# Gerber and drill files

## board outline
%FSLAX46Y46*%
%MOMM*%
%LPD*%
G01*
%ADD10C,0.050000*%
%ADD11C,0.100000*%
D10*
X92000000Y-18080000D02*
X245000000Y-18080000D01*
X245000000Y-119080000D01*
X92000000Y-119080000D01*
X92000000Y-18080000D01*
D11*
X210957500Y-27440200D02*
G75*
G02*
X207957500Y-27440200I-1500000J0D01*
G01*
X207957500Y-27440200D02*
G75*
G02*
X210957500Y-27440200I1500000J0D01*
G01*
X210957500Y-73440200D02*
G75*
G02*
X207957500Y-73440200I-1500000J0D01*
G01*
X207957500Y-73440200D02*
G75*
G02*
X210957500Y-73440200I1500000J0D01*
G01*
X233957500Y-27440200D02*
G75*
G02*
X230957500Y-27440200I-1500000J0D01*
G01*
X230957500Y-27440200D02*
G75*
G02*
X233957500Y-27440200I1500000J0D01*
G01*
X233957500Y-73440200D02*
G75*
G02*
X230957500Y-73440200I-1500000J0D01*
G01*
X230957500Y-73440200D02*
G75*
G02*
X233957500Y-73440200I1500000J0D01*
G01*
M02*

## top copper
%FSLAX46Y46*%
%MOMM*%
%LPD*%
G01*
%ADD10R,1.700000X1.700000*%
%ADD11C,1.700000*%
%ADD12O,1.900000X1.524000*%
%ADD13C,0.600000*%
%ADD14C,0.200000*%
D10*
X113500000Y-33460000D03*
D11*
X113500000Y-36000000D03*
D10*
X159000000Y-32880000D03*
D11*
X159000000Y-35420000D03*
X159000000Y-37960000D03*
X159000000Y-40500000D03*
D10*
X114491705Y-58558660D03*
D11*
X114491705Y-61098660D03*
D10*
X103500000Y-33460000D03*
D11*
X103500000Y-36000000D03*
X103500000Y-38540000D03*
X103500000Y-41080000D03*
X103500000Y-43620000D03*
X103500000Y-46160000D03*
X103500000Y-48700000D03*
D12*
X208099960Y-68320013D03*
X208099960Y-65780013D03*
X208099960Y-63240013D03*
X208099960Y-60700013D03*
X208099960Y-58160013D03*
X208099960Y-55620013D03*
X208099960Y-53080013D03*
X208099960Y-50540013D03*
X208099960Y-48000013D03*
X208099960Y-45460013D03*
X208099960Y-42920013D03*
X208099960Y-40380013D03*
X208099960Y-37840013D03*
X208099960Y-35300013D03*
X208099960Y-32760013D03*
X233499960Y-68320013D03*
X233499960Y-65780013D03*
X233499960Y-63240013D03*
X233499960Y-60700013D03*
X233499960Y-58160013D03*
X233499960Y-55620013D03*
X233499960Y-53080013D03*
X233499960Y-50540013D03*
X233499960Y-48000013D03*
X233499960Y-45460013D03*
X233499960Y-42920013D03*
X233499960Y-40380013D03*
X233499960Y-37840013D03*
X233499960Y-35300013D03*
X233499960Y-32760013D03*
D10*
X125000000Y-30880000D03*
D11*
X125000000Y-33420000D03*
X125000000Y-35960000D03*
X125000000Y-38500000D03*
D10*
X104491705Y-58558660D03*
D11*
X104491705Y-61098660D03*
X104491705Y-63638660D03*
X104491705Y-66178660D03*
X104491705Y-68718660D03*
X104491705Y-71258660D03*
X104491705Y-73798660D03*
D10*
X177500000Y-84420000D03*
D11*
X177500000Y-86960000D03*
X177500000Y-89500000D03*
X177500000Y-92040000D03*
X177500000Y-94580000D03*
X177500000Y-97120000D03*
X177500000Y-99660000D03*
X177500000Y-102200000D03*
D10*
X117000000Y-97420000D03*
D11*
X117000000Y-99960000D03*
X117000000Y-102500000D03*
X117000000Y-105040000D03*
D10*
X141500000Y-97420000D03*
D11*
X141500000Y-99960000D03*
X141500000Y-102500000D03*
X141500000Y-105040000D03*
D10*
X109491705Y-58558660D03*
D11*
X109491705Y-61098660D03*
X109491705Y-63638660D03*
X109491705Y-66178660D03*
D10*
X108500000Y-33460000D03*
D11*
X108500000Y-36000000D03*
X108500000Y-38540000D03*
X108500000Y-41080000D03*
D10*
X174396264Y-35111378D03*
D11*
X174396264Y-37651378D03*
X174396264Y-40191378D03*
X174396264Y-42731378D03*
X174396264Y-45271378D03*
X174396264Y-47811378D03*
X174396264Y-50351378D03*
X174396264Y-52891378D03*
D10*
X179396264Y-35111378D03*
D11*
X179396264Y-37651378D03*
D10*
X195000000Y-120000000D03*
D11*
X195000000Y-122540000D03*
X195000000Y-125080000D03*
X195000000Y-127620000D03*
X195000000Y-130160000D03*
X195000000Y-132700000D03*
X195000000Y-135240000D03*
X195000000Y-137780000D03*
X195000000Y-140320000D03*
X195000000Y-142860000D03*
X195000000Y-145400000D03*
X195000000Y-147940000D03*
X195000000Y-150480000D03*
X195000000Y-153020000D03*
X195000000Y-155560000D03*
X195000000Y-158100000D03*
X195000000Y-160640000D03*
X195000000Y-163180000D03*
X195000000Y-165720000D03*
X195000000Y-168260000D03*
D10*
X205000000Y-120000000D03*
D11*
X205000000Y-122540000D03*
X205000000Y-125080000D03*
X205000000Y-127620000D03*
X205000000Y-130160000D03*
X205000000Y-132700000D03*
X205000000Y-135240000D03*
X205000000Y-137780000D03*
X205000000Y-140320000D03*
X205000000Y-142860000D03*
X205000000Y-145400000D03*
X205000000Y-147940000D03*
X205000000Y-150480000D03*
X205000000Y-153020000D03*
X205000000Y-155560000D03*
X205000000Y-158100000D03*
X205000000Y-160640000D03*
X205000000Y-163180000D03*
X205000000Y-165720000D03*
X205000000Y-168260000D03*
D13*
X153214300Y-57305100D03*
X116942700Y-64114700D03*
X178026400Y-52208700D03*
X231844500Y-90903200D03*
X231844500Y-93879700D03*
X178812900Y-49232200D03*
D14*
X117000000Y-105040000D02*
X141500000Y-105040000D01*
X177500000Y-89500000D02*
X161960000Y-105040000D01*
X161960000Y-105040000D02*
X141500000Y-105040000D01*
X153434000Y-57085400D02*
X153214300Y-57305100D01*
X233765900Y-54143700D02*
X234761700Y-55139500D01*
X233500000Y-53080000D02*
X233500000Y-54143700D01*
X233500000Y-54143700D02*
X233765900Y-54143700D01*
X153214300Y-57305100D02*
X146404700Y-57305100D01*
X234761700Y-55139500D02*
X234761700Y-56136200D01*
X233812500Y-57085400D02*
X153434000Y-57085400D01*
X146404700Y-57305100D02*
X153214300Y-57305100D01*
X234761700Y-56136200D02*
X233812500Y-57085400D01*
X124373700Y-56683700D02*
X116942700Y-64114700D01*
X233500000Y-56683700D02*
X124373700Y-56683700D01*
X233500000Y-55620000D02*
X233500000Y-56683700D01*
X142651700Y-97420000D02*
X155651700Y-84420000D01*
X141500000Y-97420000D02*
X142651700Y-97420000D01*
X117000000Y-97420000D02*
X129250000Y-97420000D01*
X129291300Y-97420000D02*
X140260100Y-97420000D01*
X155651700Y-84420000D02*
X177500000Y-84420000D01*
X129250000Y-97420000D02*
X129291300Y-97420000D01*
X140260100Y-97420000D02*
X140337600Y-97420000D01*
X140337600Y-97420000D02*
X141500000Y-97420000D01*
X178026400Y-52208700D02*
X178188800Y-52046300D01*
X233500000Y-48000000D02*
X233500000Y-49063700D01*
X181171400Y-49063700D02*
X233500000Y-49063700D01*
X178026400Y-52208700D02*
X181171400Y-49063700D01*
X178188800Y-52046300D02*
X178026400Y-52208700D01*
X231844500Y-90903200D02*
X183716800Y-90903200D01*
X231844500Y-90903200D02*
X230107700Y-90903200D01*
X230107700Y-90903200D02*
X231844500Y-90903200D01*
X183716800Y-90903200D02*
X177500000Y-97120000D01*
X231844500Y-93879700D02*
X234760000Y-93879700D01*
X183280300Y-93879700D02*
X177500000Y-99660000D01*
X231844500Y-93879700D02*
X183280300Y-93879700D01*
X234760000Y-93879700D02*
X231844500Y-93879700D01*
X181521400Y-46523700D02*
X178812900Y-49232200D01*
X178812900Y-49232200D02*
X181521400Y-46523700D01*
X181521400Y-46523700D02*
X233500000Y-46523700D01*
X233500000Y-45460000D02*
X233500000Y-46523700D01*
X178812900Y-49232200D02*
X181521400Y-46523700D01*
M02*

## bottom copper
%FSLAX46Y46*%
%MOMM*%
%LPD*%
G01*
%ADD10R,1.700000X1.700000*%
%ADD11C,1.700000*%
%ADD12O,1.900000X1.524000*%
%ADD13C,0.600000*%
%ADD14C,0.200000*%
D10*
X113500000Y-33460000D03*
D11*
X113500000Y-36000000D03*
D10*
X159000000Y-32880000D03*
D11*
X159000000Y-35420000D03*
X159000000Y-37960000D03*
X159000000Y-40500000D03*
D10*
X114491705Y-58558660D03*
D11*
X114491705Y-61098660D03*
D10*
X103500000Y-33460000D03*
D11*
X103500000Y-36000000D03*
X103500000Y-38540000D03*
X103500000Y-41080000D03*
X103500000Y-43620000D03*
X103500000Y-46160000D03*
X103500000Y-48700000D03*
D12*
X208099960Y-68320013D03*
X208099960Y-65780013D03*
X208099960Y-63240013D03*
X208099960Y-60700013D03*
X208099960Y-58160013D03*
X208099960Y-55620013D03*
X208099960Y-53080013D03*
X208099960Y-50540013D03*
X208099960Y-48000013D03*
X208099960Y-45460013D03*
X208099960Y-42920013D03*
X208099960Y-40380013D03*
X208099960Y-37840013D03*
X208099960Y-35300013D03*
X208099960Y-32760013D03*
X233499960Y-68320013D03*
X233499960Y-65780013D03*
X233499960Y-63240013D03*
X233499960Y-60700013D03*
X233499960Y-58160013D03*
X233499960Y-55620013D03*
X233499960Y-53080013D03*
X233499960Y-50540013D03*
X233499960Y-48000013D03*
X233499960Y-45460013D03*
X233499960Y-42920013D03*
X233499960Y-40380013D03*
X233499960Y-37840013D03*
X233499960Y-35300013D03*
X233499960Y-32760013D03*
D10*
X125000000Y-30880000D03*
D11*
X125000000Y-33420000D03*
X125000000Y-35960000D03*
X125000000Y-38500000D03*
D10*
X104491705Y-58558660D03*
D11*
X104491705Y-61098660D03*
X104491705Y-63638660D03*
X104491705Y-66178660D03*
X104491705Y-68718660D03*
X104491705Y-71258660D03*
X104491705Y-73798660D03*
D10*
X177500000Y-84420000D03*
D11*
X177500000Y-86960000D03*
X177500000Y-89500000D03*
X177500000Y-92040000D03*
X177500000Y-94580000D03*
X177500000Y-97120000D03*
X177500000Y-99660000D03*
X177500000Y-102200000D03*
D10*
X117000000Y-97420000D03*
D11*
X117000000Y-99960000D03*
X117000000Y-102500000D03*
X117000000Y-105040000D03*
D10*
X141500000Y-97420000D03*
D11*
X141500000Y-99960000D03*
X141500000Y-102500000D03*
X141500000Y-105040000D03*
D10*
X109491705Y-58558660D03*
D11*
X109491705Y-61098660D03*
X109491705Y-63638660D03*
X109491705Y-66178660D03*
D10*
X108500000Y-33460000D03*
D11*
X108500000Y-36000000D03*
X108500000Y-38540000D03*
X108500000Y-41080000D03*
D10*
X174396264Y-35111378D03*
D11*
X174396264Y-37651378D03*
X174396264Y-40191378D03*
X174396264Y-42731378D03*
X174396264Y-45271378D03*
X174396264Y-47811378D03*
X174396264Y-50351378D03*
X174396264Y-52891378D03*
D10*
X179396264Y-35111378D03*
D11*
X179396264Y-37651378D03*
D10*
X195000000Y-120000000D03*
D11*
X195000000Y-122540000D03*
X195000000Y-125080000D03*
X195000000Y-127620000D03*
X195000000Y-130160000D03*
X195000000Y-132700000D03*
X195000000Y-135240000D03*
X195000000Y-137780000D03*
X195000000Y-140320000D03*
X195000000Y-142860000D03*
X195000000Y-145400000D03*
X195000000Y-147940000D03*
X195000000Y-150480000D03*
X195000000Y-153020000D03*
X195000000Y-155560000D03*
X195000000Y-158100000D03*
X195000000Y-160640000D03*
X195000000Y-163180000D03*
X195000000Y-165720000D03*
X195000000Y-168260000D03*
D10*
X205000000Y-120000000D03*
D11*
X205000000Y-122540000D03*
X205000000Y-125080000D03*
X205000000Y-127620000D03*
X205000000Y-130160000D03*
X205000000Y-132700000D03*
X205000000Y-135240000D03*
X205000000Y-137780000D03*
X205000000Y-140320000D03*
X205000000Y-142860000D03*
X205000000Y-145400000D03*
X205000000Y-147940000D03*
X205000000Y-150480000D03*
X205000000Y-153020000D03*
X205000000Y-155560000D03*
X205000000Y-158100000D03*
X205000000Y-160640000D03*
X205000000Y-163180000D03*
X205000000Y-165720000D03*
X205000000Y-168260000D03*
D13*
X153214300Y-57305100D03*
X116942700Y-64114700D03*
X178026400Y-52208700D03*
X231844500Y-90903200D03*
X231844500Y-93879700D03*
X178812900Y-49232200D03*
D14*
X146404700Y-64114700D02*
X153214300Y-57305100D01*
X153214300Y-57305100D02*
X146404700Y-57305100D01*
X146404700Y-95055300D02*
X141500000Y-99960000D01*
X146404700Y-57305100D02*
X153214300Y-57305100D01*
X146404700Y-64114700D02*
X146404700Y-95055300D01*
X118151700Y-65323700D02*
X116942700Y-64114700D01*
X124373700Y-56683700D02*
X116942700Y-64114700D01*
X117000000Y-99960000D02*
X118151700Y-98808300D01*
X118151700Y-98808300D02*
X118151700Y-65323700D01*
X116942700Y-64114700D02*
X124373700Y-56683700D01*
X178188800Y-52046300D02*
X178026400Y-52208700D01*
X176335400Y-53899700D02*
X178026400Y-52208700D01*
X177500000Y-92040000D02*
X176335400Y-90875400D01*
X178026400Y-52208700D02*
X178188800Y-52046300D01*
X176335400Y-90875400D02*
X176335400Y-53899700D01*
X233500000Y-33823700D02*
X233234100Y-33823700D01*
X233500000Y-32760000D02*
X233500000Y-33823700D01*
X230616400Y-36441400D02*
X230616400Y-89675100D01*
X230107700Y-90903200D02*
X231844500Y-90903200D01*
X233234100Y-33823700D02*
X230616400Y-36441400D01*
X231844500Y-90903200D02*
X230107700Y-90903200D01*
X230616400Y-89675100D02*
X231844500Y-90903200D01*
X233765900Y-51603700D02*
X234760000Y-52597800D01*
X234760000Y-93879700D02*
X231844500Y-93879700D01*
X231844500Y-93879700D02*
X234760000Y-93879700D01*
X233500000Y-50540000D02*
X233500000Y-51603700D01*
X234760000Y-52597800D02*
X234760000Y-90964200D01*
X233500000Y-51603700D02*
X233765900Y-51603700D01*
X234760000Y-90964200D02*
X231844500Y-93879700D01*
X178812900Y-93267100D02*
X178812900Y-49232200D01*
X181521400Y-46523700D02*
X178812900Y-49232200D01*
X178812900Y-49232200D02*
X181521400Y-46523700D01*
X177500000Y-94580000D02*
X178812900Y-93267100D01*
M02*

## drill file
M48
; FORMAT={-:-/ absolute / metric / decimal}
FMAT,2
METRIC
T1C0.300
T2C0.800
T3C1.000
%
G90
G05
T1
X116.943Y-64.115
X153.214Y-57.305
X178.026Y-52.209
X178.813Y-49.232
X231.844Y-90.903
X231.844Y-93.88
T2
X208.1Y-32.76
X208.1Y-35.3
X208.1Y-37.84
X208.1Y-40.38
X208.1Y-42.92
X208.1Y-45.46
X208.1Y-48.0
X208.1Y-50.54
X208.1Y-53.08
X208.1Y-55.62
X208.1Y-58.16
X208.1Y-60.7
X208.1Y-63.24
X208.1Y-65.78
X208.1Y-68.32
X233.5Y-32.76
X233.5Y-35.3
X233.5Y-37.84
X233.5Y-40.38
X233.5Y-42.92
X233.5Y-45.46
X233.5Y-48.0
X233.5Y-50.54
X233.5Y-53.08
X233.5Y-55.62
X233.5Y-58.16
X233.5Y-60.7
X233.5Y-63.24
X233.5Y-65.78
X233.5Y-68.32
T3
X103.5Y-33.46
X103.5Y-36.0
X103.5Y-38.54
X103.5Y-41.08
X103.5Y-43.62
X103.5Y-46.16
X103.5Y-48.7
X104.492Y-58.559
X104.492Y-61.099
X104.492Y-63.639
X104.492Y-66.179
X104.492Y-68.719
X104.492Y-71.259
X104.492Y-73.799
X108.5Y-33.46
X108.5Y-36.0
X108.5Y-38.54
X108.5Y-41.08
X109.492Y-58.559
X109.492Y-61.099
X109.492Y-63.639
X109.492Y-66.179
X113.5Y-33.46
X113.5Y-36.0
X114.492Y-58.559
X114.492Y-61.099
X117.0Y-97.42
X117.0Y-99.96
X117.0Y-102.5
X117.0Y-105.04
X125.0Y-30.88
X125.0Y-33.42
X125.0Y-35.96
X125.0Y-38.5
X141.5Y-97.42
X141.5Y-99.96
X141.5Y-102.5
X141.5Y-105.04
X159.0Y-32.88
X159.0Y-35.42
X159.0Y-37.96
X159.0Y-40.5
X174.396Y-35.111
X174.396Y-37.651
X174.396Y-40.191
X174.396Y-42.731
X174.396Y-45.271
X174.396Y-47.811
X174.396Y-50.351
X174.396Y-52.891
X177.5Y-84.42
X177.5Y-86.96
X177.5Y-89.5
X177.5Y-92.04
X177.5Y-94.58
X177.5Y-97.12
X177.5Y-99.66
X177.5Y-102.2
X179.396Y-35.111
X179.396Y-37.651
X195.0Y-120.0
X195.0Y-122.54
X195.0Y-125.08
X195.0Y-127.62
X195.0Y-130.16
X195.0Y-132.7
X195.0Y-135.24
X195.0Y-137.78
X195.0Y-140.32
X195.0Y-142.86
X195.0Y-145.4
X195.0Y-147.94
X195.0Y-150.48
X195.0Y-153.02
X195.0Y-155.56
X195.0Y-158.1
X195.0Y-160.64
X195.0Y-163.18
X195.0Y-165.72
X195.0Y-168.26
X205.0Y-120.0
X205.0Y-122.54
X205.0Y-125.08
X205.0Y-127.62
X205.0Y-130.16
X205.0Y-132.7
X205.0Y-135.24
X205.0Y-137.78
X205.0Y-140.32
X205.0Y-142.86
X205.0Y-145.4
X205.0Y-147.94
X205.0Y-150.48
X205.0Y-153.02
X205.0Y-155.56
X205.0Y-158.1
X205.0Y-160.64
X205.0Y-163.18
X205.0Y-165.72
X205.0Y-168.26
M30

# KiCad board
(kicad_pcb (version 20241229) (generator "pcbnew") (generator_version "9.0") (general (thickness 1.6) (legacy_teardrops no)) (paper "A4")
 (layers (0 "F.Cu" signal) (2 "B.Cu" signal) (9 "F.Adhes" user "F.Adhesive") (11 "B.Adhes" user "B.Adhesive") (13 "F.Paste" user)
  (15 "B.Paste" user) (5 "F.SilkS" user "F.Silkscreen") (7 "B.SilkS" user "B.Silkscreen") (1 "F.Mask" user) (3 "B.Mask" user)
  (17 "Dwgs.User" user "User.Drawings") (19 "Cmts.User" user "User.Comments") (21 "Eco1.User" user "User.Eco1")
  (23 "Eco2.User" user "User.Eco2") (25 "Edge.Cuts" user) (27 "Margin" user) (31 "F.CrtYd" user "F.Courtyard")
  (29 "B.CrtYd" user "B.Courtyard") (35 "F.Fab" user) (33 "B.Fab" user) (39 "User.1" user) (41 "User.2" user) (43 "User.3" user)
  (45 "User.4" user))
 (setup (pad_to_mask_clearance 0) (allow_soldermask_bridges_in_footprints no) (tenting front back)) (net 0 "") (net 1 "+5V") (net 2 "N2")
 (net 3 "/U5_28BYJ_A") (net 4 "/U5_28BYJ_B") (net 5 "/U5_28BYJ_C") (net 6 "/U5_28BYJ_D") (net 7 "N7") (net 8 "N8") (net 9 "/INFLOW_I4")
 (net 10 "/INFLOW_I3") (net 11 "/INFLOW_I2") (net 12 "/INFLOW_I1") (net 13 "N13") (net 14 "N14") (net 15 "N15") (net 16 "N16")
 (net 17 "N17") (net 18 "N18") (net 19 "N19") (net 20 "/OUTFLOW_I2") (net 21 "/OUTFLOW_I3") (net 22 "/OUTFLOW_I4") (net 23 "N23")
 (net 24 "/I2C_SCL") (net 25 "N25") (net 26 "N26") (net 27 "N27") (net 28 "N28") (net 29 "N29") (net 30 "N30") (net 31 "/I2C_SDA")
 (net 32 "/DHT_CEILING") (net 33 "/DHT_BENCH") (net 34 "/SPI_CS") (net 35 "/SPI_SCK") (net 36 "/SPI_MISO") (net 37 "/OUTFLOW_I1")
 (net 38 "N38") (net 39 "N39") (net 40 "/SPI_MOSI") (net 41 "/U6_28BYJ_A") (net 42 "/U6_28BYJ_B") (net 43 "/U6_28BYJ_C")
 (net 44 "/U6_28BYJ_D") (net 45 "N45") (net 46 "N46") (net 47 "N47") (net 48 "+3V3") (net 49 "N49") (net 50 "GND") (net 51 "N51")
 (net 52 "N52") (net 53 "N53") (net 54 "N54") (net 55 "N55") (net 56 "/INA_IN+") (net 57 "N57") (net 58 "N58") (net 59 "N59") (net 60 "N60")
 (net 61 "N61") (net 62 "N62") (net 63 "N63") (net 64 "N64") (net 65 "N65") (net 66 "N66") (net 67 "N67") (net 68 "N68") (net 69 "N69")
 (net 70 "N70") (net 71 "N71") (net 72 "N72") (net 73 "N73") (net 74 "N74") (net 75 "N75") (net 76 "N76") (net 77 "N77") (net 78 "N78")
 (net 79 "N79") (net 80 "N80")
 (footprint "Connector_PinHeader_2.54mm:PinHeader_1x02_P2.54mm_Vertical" (layer "F.Cu") (at 113.5 33.46)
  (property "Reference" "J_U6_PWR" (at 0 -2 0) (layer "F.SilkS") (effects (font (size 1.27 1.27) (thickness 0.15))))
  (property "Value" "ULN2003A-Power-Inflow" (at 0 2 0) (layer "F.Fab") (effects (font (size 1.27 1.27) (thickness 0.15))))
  (pad "1" thru_hole rect (at 0 0.00) (size 1.7 1.7) (drill 1) (layers "*.Cu" "*.Mask") (remove_unused_layers no) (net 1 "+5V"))
  (pad "2" thru_hole circle (at 0 2.54) (size 1.7 1.7) (drill 1) (layers "*.Cu" "*.Mask") (remove_unused_layers no) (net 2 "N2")))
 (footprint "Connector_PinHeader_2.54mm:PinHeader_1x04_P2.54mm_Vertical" (layer "F.Cu") (at 159 32.88)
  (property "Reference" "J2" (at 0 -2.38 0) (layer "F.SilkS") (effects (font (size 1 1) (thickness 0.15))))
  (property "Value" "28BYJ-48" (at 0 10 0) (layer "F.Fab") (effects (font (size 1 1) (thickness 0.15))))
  (pad "1" thru_hole rect (at 0 0) (size 1.7 1.7) (drill 1) (layers "*.Cu" "*.Mask") (remove_unused_layers no) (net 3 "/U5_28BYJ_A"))
  (pad "2" thru_hole circle (at 0 2.54) (size 1.7 1.7) (drill 1) (layers "*.Cu" "*.Mask") (remove_unused_layers no) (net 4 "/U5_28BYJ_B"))
  (pad "3" thru_hole circle (at 0 5.08) (size 1.7 1.7) (drill 1) (layers "*.Cu" "*.Mask") (remove_unused_layers no) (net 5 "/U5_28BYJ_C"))
  (pad "4" thru_hole circle (at 0 7.62) (size 1.7 1.7) (drill 1) (layers "*.Cu" "*.Mask") (remove_unused_layers no) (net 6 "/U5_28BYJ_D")))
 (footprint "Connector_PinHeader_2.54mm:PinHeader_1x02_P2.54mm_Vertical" (layer "F.Cu") (at 114.491705 58.55866)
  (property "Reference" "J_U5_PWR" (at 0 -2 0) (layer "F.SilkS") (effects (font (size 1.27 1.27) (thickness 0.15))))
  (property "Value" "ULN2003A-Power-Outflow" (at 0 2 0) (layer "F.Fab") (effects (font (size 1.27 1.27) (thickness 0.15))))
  (pad "1" thru_hole rect (at 0 0.00) (size 1.7 1.7) (drill 1) (layers "*.Cu" "*.Mask") (remove_unused_layers no) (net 1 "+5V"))
  (pad "2" thru_hole circle (at 0 2.54) (size 1.7 1.7) (drill 1) (layers "*.Cu" "*.Mask") (remove_unused_layers no) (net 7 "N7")))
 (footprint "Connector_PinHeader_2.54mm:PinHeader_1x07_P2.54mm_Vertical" (layer "F.Cu") (at 103.5 33.46)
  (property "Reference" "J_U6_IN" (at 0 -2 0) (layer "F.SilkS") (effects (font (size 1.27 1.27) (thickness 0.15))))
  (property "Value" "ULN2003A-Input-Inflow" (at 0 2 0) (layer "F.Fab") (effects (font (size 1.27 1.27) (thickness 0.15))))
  (pad "1" thru_hole rect (at 0 0.00) (size 1.7 1.7) (drill 1) (layers "*.Cu" "*.Mask") (remove_unused_layers no) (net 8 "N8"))
  (pad "2" thru_hole circle (at 0 2.54) (size 1.7 1.7) (drill 1) (layers "*.Cu" "*.Mask") (remove_unused_layers no) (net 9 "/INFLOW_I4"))
  (pad "3" thru_hole circle (at 0 5.08) (size 1.7 1.7) (drill 1) (layers "*.Cu" "*.Mask") (remove_unused_layers no) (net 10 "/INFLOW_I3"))
  (pad "4" thru_hole circle (at 0 7.62) (size 1.7 1.7) (drill 1) (layers "*.Cu" "*.Mask") (remove_unused_layers no) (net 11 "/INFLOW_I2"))
  (pad "5" thru_hole circle (at 0 10.16) (size 1.7 1.7) (drill 1) (layers "*.Cu" "*.Mask") (remove_unused_layers no) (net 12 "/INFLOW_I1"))
  (pad "6" thru_hole circle (at 0 12.70) (size 1.7 1.7) (drill 1) (layers "*.Cu" "*.Mask") (remove_unused_layers no) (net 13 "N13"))
  (pad "7" thru_hole circle (at 0 15.24) (size 1.7 1.7) (drill 1) (layers "*.Cu" "*.Mask") (remove_unused_layers no) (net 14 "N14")))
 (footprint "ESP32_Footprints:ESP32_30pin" (layer "F.Cu") (at 220.0275 51.3002)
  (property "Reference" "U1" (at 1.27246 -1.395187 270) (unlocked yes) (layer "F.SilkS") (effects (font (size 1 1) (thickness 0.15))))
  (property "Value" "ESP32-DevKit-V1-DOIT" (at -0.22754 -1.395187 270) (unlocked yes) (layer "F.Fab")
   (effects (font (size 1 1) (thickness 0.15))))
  (fp_circle (center -10.57 -23.86) (end -10.57 -22.36) (stroke (width 0.1) (type default)) (fill no) (layer "Edge.Cuts"))
  (fp_circle (center -10.57 22.14) (end -10.57 23.64) (stroke (width 0.1) (type default)) (fill no) (layer "Edge.Cuts"))
  (fp_circle (center 12.43 -23.86) (end 12.43 -22.36) (stroke (width 0.1) (type default)) (fill no) (layer "Edge.Cuts"))
  (fp_circle (center 12.43 22.14) (end 12.43 23.64) (stroke (width 0.1) (type default)) (fill no) (layer "Edge.Cuts"))
  (pad "1" thru_hole oval (at -11.92754 17.019813 270) (size 1.524 1.9) (drill 0.8) (layers "*.Cu" "*.Mask") (remove_unused_layers no)
   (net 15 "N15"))
  (pad "2" thru_hole oval (at -11.92754 14.479813 270) (size 1.524 1.9) (drill 0.8) (layers "*.Cu" "*.Mask") (remove_unused_layers no)
   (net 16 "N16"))
  (pad "3" thru_hole oval (at -11.92754 11.939813 270) (size 1.524 1.9) (drill 0.8) (layers "*.Cu" "*.Mask") (remove_unused_layers no)
   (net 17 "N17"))
  (pad "4" thru_hole oval (at -11.92754 9.399813 270) (size 1.524 1.9) (drill 0.8) (layers "*.Cu" "*.Mask") (remove_unused_layers no)
   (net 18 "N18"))
  (pad "5" thru_hole oval (at -11.92754 6.859813 270) (size 1.524 1.9) (drill 0.8) (layers "*.Cu" "*.Mask") (remove_unused_layers no)
   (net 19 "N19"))
  (pad "6" thru_hole oval (at -11.92754 4.319813 270) (size 1.524 1.9) (drill 0.8) (layers "*.Cu" "*.Mask") (remove_unused_layers no)
   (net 10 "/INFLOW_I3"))
  (pad "7" thru_hole oval (at -11.92754 1.779813 270) (size 1.524 1.9) (drill 0.8) (layers "*.Cu" "*.Mask") (remove_unused_layers no)
   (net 9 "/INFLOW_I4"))
  (pad "8" thru_hole oval (at -11.92754 -0.760187 270) (size 1.524 1.9) (drill 0.8) (layers "*.Cu" "*.Mask") (remove_unused_layers no)
   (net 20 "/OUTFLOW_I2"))
  (pad "9" thru_hole oval (at -11.92754 -3.300187 270) (size 1.524 1.9) (drill 0.8) (layers "*.Cu" "*.Mask") (remove_unused_layers no)
   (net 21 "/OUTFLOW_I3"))
  (pad "10" thru_hole oval (at -11.92754 -5.840187 270) (size 1.524 1.9) (drill 0.8) (layers "*.Cu" "*.Mask") (remove_unused_layers no)
   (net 11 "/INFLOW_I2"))
  (pad "11" thru_hole oval (at -11.92754 -8.380187 270) (size 1.524 1.9) (drill 0.8) (layers "*.Cu" "*.Mask") (remove_unused_layers no)
   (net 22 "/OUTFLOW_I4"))
  (pad "12" thru_hole oval (at -11.92754 -10.920187 270) (size 1.524 1.9) (drill 0.8) (layers "*.Cu" "*.Mask") (remove_unused_layers no)
   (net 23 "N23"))
  (pad "13" thru_hole oval (at -11.92754 -13.460187 270) (size 1.524 1.9) (drill 0.8) (layers "*.Cu" "*.Mask") (remove_unused_layers no)
   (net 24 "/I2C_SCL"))
  (pad "14" thru_hole oval (at -11.92754 -16.000187 270) (size 1.524 1.9) (drill 0.8) (layers "*.Cu" "*.Mask") (remove_unused_layers no)
   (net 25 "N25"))
  (pad "15" thru_hole oval (at -11.92754 -18.540187 270) (size 1.524 1.9) (drill 0.8) (layers "*.Cu" "*.Mask") (remove_unused_layers no)
   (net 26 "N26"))
  (pad "16" thru_hole oval (at 13.47246 17.019813 270) (size 1.524 1.9) (drill 0.8) (layers "*.Cu" "*.Mask") (remove_unused_layers no)
   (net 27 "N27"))
  (pad "17" thru_hole oval (at 13.47246 14.479813 270) (size 1.524 1.9) (drill 0.8) (layers "*.Cu" "*.Mask") (remove_unused_layers no)
   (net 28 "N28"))
  (pad "18" thru_hole oval (at 13.47246 11.939813 270) (size 1.524 1.9) (drill 0.8) (layers "*.Cu" "*.Mask") (remove_unused_layers no)
   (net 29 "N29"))
  (pad "19" thru_hole oval (at 13.47246 9.399813 270) (size 1.524 1.9) (drill 0.8) (layers "*.Cu" "*.Mask") (remove_unused_layers no)
   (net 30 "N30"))
  (pad "20" thru_hole oval (at 13.47246 6.859813 270) (size 1.524 1.9) (drill 0.8) (layers "*.Cu" "*.Mask" "Dwgs.User")
   (remove_unused_layers no) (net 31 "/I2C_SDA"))
  (pad "21" thru_hole oval (at 13.47246 4.319813 270) (size 1.524 1.9) (drill 0.8) (layers "*.Cu" "*.Mask") (remove_unused_layers no)
   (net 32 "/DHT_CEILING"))
  (pad "22" thru_hole oval (at 13.47246 1.779813 270) (size 1.524 1.9) (drill 0.8) (layers "*.Cu" "*.Mask") (remove_unused_layers no)
   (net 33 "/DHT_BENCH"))
  (pad "23" thru_hole oval (at 13.47246 -0.760187 270) (size 1.524 1.9) (drill 0.8) (layers "*.Cu" "*.Mask") (remove_unused_layers no)
   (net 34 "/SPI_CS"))
  (pad "24" thru_hole oval (at 13.47246 -3.300187 270) (size 1.524 1.9) (drill 0.8) (layers "*.Cu" "*.Mask") (remove_unused_layers no)
   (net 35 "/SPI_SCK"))
  (pad "25" thru_hole oval (at 13.47246 -5.840187 270) (size 1.524 1.9) (drill 0.8) (layers "*.Cu" "*.Mask") (remove_unused_layers no)
   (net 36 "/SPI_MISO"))
  (pad "26" thru_hole oval (at 13.47246 -8.380187 270) (size 1.524 1.9) (drill 0.8) (layers "*.Cu" "*.Mask") (remove_unused_layers no)
   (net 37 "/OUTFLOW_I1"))
  (pad "27" thru_hole oval (at 13.47246 -10.920187 270) (size 1.524 1.9) (drill 0.8) (layers "*.Cu" "*.Mask") (remove_unused_layers no)
   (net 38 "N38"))
  (pad "28" thru_hole oval (at 13.47246 -13.460187 270) (size 1.524 1.9) (drill 0.8) (layers "*.Cu" "*.Mask") (remove_unused_layers no)
   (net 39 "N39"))
  (pad "29" thru_hole oval (at 13.47246 -16.000187 270) (size 1.524 1.9) (drill 0.8) (layers "*.Cu" "*.Mask") (remove_unused_layers no)
   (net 12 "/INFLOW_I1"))
  (pad "30" thru_hole oval (at 13.47246 -18.540187 270) (size 1.524 1.9) (drill 0.8) (layers "*.Cu" "*.Mask") (remove_unused_layers no)
   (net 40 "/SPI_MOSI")))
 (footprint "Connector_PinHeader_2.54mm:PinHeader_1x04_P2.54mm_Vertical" (layer "F.Cu") (at 125 30.88)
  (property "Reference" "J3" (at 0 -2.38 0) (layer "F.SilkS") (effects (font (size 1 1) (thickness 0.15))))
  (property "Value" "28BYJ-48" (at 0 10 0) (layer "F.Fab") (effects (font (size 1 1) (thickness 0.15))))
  (pad "1" thru_hole rect (at 0 0) (size 1.7 1.7) (drill 1) (layers "*.Cu" "*.Mask") (remove_unused_layers no) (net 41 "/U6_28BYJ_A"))
  (pad "2" thru_hole circle (at 0 2.54) (size 1.7 1.7) (drill 1) (layers "*.Cu" "*.Mask") (remove_unused_layers no) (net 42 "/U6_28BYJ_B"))
  (pad "3" thru_hole circle (at 0 5.08) (size 1.7 1.7) (drill 1) (layers "*.Cu" "*.Mask") (remove_unused_layers no) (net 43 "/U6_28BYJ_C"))
  (pad "4" thru_hole circle (at 0 7.62) (size 1.7 1.7) (drill 1) (layers "*.Cu" "*.Mask") (remove_unused_layers no) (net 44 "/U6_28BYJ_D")))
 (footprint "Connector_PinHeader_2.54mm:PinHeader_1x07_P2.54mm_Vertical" (layer "F.Cu") (at 104.491705 58.55866)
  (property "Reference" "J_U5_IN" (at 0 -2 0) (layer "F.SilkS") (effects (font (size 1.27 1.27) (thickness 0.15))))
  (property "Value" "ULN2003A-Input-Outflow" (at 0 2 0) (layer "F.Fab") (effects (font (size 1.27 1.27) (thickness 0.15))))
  (pad "1" thru_hole rect (at 0 0.00) (size 1.7 1.7) (drill 1) (layers "*.Cu" "*.Mask") (remove_unused_layers no) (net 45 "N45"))
  (pad "2" thru_hole circle (at 0 2.54) (size 1.7 1.7) (drill 1) (layers "*.Cu" "*.Mask") (remove_unused_layers no) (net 22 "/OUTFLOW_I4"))
  (pad "3" thru_hole circle (at 0 5.08) (size 1.7 1.7) (drill 1) (layers "*.Cu" "*.Mask") (remove_unused_layers no) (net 21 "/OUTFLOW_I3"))
  (pad "4" thru_hole circle (at 0 7.62) (size 1.7 1.7) (drill 1) (layers "*.Cu" "*.Mask") (remove_unused_layers no) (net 20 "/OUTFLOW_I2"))
  (pad "5" thru_hole circle (at 0 10.16) (size 1.7 1.7) (drill 1) (layers "*.Cu" "*.Mask") (remove_unused_layers no) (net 37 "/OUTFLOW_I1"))
  (pad "6" thru_hole circle (at 0 12.70) (size 1.7 1.7) (drill 1) (layers "*.Cu" "*.Mask") (remove_unused_layers no) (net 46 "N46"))
  (pad "7" thru_hole circle (at 0 15.24) (size 1.7 1.7) (drill 1) (layers "*.Cu" "*.Mask") (remove_unused_layers no) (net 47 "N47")))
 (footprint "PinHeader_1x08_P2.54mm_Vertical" (layer "F.Cu") (at 177.5 84.42)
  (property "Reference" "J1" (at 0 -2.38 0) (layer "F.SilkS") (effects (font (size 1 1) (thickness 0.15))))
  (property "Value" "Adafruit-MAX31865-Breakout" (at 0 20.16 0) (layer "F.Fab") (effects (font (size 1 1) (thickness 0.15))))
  (pad "1" thru_hole rect (at 0 0) (size 1.7 1.7) (drill 1) (layers "*.Cu" "*.Mask") (remove_unused_layers no) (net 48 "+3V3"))
  (pad "2" thru_hole circle (at 0 2.54) (size 1.7 1.7) (drill 1) (layers "*.Cu" "*.Mask") (remove_unused_layers no) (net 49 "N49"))
  (pad "3" thru_hole circle (at 0 5.08) (size 1.7 1.7) (drill 1) (layers "*.Cu" "*.Mask") (remove_unused_layers no) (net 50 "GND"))
  (pad "4" thru_hole circle (at 0 7.62) (size 1.7 1.7) (drill 1) (layers "*.Cu" "*.Mask") (remove_unused_layers no) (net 35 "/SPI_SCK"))
  (pad "5" thru_hole circle (at 0 10.16) (size 1.7 1.7) (drill 1) (layers "*.Cu" "*.Mask") (remove_unused_layers no) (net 36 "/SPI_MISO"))
  (pad "6" thru_hole circle (at 0 12.7) (size 1.7 1.7) (drill 1) (layers "*.Cu" "*.Mask") (remove_unused_layers no) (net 40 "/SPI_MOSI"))
  (pad "7" thru_hole circle (at 0 15.24) (size 1.7 1.7) (drill 1) (layers "*.Cu" "*.Mask") (remove_unused_layers no) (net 34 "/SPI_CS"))
  (pad "8" thru_hole circle (at 0 17.78) (size 1.7 1.7) (drill 1) (layers "*.Cu" "*.Mask") (remove_unused_layers no) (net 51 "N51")))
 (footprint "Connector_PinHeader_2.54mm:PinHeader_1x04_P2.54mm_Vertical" (layer "F.Cu") (at 117 97.42)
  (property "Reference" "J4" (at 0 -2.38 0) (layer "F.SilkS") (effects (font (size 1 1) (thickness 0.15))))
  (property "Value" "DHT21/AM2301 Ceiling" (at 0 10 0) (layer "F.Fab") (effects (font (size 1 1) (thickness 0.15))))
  (pad "1" thru_hole rect (at 0 0) (size 1.7 1.7) (drill 1) (layers "*.Cu" "*.Mask") (remove_unused_layers no) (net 48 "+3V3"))
  (pad "2" thru_hole circle (at 0 2.54) (size 1.7 1.7) (drill 1) (layers "*.Cu" "*.Mask") (remove_unused_layers no) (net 32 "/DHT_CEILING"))
  (pad "3" thru_hole circle (at 0 5.08) (size 1.7 1.7) (drill 1) (layers "*.Cu" "*.Mask") (remove_unused_layers no) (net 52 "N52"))
  (pad "4" thru_hole circle (at 0 7.62) (size 1.7 1.7) (drill 1) (layers "*.Cu" "*.Mask") (remove_unused_layers no) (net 50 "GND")))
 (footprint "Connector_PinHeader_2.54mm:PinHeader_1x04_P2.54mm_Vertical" (layer "F.Cu") (at 141.5 97.42)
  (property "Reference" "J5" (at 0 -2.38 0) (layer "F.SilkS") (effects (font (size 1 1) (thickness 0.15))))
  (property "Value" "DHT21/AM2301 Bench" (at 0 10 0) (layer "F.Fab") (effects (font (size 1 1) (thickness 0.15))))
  (pad "1" thru_hole rect (at 0 0) (size 1.7 1.7) (drill 1) (layers "*.Cu" "*.Mask") (remove_unused_layers no) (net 48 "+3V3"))
  (pad "2" thru_hole circle (at 0 2.54) (size 1.7 1.7) (drill 1) (layers "*.Cu" "*.Mask") (remove_unused_layers no) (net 33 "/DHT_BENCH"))
  (pad "3" thru_hole circle (at 0 5.08) (size 1.7 1.7) (drill 1) (layers "*.Cu" "*.Mask") (remove_unused_layers no) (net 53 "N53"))
  (pad "4" thru_hole circle (at 0 7.62) (size 1.7 1.7) (drill 1) (layers "*.Cu" "*.Mask") (remove_unused_layers no) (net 50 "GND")))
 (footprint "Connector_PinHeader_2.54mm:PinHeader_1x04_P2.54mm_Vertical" (layer "F.Cu") (at 109.491705 58.55866)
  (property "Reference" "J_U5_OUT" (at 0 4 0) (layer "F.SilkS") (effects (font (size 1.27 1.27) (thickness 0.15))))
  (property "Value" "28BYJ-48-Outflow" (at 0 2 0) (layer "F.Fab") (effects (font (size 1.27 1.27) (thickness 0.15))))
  (pad "1" thru_hole rect (at 0 0.00) (size 1.7 1.7) (drill 1) (layers "*.Cu" "*.Mask") (remove_unused_layers no) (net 5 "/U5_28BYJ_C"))
  (pad "2" thru_hole circle (at 0 2.54) (size 1.7 1.7) (drill 1) (layers "*.Cu" "*.Mask") (remove_unused_layers no) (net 4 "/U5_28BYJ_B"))
  (pad "3" thru_hole circle (at 0 5.08) (size 1.7 1.7) (drill 1) (layers "*.Cu" "*.Mask") (remove_unused_layers no) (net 3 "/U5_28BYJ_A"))
  (pad "4" thru_hole circle (at 0 7.62) (size 1.7 1.7) (drill 1) (layers "*.Cu" "*.Mask") (remove_unused_layers no) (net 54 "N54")))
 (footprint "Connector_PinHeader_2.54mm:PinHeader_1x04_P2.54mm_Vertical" (layer "F.Cu") (at 108.5 33.46)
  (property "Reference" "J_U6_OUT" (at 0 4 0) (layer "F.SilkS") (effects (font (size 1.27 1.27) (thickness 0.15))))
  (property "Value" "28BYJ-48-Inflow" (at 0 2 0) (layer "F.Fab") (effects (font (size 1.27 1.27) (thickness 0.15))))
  (pad "1" thru_hole rect (at 0 0.00) (size 1.7 1.7) (drill 1) (layers "*.Cu" "*.Mask") (remove_unused_layers no) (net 43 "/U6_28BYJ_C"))
  (pad "2" thru_hole circle (at 0 2.54) (size 1.7 1.7) (drill 1) (layers "*.Cu" "*.Mask") (remove_unused_layers no) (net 42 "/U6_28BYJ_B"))
  (pad "3" thru_hole circle (at 0 5.08) (size 1.7 1.7) (drill 1) (layers "*.Cu" "*.Mask") (remove_unused_layers no) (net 41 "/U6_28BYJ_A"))
  (pad "4" thru_hole circle (at 0 7.62) (size 1.7 1.7) (drill 1) (layers "*.Cu" "*.Mask") (remove_unused_layers no) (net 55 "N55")))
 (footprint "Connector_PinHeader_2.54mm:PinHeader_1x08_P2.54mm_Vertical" (layer "F.Cu") (at 174.396264 35.111378)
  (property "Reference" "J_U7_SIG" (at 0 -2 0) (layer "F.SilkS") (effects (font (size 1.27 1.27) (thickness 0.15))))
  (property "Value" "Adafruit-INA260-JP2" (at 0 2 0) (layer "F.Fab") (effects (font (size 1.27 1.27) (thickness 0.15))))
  (pad "1" thru_hole rect (at 0 0.00) (size 1.7 1.7) (drill 1) (layers "*.Cu" "*.Mask") (remove_unused_layers no) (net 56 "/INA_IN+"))
  (pad "2" thru_hole circle (at 0 2.54) (size 1.7 1.7) (drill 1) (layers "*.Cu" "*.Mask") (remove_unused_layers no) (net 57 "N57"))
  (pad "3" thru_hole circle (at 0 5.08) (size 1.7 1.7) (drill 1) (layers "*.Cu" "*.Mask") (remove_unused_layers no) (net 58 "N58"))
  (pad "4" thru_hole circle (at 0 7.62) (size 1.7 1.7) (drill 1) (layers "*.Cu" "*.Mask") (remove_unused_layers no) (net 31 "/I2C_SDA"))
  (pad "5" thru_hole circle (at 0 10.16) (size 1.7 1.7) (drill 1) (layers "*.Cu" "*.Mask") (remove_unused_layers no) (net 24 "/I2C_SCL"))
  (pad "6" thru_hole circle (at 0 12.70) (size 1.7 1.7) (drill 1) (layers "*.Cu" "*.Mask") (remove_unused_layers no) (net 50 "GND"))
  (pad "7" thru_hole circle (at 0 15.24) (size 1.7 1.7) (drill 1) (layers "*.Cu" "*.Mask") (remove_unused_layers no) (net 48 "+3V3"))
  (pad "8" thru_hole circle (at 0 17.78) (size 1.7 1.7) (drill 1) (layers "*.Cu" "*.Mask") (remove_unused_layers no) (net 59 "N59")))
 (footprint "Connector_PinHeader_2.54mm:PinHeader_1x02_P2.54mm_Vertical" (layer "F.Cu") (at 179.396264 35.111378)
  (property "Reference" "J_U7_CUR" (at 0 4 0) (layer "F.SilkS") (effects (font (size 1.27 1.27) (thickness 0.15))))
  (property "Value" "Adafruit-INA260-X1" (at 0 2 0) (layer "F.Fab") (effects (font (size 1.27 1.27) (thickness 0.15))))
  (pad "1" thru_hole rect (at 0 0.00) (size 1.7 1.7) (drill 1) (layers "*.Cu" "*.Mask") (remove_unused_layers no) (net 56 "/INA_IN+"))
  (pad "2" thru_hole circle (at 0 2.54) (size 1.7 1.7) (drill 1) (layers "*.Cu" "*.Mask") (remove_unused_layers no) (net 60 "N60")))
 (gr_rect (start 92 18.08) (end 245 119.08) (stroke (width 0.05) (type default)) (fill no) (layer "Edge.Cuts"))
 (segment (start 117 105.04) (end 141.5 105.04) (width 0.2) (layer "F.Cu") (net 50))
 (segment (start 177.5 89.5) (end 161.96 105.04) (width 0.2) (layer "F.Cu") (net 50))
 (segment (start 161.96 105.04) (end 141.5 105.04) (width 0.2) (layer "F.Cu") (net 50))
 (segment (start 153.434 57.0854) (end 153.2143 57.3051) (width 0.2) (layer "F.Cu") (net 33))
 (segment (start 233.7659 54.1437) (end 234.7617 55.1395) (width 0.2) (layer "F.Cu") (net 33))
 (segment (start 233.5 53.08) (end 233.5 54.1437) (width 0.2) (layer "F.Cu") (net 33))
 (segment (start 233.5 54.1437) (end 233.7659 54.1437) (width 0.2) (layer "F.Cu") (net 33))
 (segment (start 153.2143 57.3051) (end 146.4047 57.3051) (width 0.2) (layer "F.Cu") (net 33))
 (segment (start 234.7617 55.1395) (end 234.7617 56.1362) (width 0.2) (layer "F.Cu") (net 33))
 (segment (start 233.8125 57.0854) (end 153.434 57.0854) (width 0.2) (layer "F.Cu") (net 33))
 (segment (start 146.4047 57.3051) (end 153.2143 57.3051) (width 0.2) (layer "F.Cu") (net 33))
 (segment (start 234.7617 56.1362) (end 233.8125 57.0854) (width 0.2) (layer "F.Cu") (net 33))
 (via (at 153.2143 57.3051) (size 0.6) (drill 0.3) (layers "F.Cu" "B.Cu") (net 33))
 (segment (start 146.4047 64.1147) (end 153.2143 57.3051) (width 0.2) (layer "B.Cu") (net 33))
 (segment (start 153.2143 57.3051) (end 146.4047 57.3051) (width 0.2) (layer "B.Cu") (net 33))
 (segment (start 146.4047 95.0553) (end 141.5 99.96) (width 0.2) (layer "B.Cu") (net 33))
 (segment (start 146.4047 57.3051) (end 153.2143 57.3051) (width 0.2) (layer "B.Cu") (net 33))
 (segment (start 146.4047 64.1147) (end 146.4047 95.0553) (width 0.2) (layer "B.Cu") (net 33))
 (segment (start 124.3737 56.6837) (end 116.9427 64.1147) (width 0.2) (layer "F.Cu") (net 32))
 (segment (start 233.5 56.6837) (end 124.3737 56.6837) (width 0.2) (layer "F.Cu") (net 32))
 (segment (start 233.5 55.62) (end 233.5 56.6837) (width 0.2) (layer "F.Cu") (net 32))
 (via (at 116.9427 64.1147) (size 0.6) (drill 0.3) (layers "F.Cu" "B.Cu") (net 32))
 (segment (start 118.1517 65.3237) (end 116.9427 64.1147) (width 0.2) (layer "B.Cu") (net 32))
 (segment (start 124.3737 56.6837) (end 116.9427 64.1147) (width 0.2) (layer "B.Cu") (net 32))
 (segment (start 117 99.96) (end 118.1517 98.8083) (width 0.2) (layer "B.Cu") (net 32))
 (segment (start 118.1517 98.8083) (end 118.1517 65.3237) (width 0.2) (layer "B.Cu") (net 32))
 (segment (start 116.9427 64.1147) (end 124.3737 56.6837) (width 0.2) (layer "B.Cu") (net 32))
 (segment (start 142.6517 97.42) (end 155.6517 84.42) (width 0.2) (layer "F.Cu") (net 48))
 (segment (start 141.5 97.42) (end 142.6517 97.42) (width 0.2) (layer "F.Cu") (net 48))
 (segment (start 117 97.42) (end 129.25 97.42) (width 0.2) (layer "F.Cu") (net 48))
 (segment (start 129.2913 97.42) (end 140.2601 97.42) (width 0.2) (layer "F.Cu") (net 48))
 (segment (start 155.6517 84.42) (end 177.5 84.42) (width 0.2) (layer "F.Cu") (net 48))
 (segment (start 129.25 97.42) (end 129.2913 97.42) (width 0.2) (layer "F.Cu") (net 48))
 (segment (start 140.2601 97.42) (end 140.3376 97.42) (width 0.2) (layer "F.Cu") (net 48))
 (segment (start 140.3376 97.42) (end 141.5 97.42) (width 0.2) (layer "F.Cu") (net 48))
 (segment (start 178.0264 52.2087) (end 178.1888 52.0463) (width 0.2) (layer "F.Cu") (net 35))
 (segment (start 233.5 48) (end 233.5 49.0637) (width 0.2) (layer "F.Cu") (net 35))
 (segment (start 181.1714 49.0637) (end 233.5 49.0637) (width 0.2) (layer "F.Cu") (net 35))
 (segment (start 178.0264 52.2087) (end 181.1714 49.0637) (width 0.2) (layer "F.Cu") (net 35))
 (segment (start 178.1888 52.0463) (end 178.0264 52.2087) (width 0.2) (layer "F.Cu") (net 35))
 (via (at 178.0264 52.2087) (size 0.6) (drill 0.3) (layers "F.Cu" "B.Cu") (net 35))
 (segment (start 178.1888 52.0463) (end 178.0264 52.2087) (width 0.2) (layer "B.Cu") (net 35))
 (segment (start 176.3354 53.8997) (end 178.0264 52.2087) (width 0.2) (layer "B.Cu") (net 35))
 (segment (start 177.5 92.04) (end 176.3354 90.8754) (width 0.2) (layer "B.Cu") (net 35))
 (segment (start 178.0264 52.2087) (end 178.1888 52.0463) (width 0.2) (layer "B.Cu") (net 35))
 (segment (start 176.3354 90.8754) (end 176.3354 53.8997) (width 0.2) (layer "B.Cu") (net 35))
 (segment (start 231.8445 90.9032) (end 183.7168 90.9032) (width 0.2) (layer "F.Cu") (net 40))
 (segment (start 231.8445 90.9032) (end 230.1077 90.9032) (width 0.2) (layer "F.Cu") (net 40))
 (segment (start 230.1077 90.9032) (end 231.8445 90.9032) (width 0.2) (layer "F.Cu") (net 40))
 (segment (start 183.7168 90.9032) (end 177.5 97.12) (width 0.2) (layer "F.Cu") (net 40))
 (via (at 231.8445 90.9032) (size 0.6) (drill 0.3) (layers "F.Cu" "B.Cu") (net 40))
 (segment (start 233.5 33.8237) (end 233.2341 33.8237) (width 0.2) (layer "B.Cu") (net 40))
 (segment (start 233.5 32.76) (end 233.5 33.8237) (width 0.2) (layer "B.Cu") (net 40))
 (segment (start 230.6164 36.4414) (end 230.6164 89.6751) (width 0.2) (layer "B.Cu") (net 40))
 (segment (start 230.1077 90.9032) (end 231.8445 90.9032) (width 0.2) (layer "B.Cu") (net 40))
 (segment (start 233.2341 33.8237) (end 230.6164 36.4414) (width 0.2) (layer "B.Cu") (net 40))
 (segment (start 231.8445 90.9032) (end 230.1077 90.9032) (width 0.2) (layer "B.Cu") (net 40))
 (segment (start 230.6164 89.6751) (end 231.8445 90.9032) (width 0.2) (layer "B.Cu") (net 40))
 (segment (start 231.8445 93.8797) (end 234.76 93.8797) (width 0.2) (layer "F.Cu") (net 34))
 (segment (start 183.2803 93.8797) (end 177.5 99.66) (width 0.2) (layer "F.Cu") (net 34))
 (segment (start 231.8445 93.8797) (end 183.2803 93.8797) (width 0.2) (layer "F.Cu") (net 34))
 (segment (start 234.76 93.8797) (end 231.8445 93.8797) (width 0.2) (layer "F.Cu") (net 34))
 (via (at 231.8445 93.8797) (size 0.6) (drill 0.3) (layers "F.Cu" "B.Cu") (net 34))
 (segment (start 233.7659 51.6037) (end 234.76 52.5978) (width 0.2) (layer "B.Cu") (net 34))
 (segment (start 234.76 93.8797) (end 231.8445 93.8797) (width 0.2) (layer "B.Cu") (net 34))
 (segment (start 231.8445 93.8797) (end 234.76 93.8797) (width 0.2) (layer "B.Cu") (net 34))
 (segment (start 233.5 50.54) (end 233.5 51.6037) (width 0.2) (layer "B.Cu") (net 34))
 (segment (start 234.76 52.5978) (end 234.76 90.9642) (width 0.2) (layer "B.Cu") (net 34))
 (segment (start 233.5 51.6037) (end 233.7659 51.6037) (width 0.2) (layer "B.Cu") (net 34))
 (segment (start 234.76 90.9642) (end 231.8445 93.8797) (width 0.2) (layer "B.Cu") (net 34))
 (segment (start 181.5214 46.5237) (end 178.8129 49.2322) (width 0.2) (layer "F.Cu") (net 36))
 (segment (start 178.8129 49.2322) (end 181.5214 46.5237) (width 0.2) (layer "F.Cu") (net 36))
 (segment (start 181.5214 46.5237) (end 233.5 46.5237) (width 0.2) (layer "F.Cu") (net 36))
 (segment (start 233.5 45.46) (end 233.5 46.5237) (width 0.2) (layer "F.Cu") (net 36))
 (segment (start 178.8129 49.2322) (end 181.5214 46.5237) (width 0.2) (layer "F.Cu") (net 36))
 (via (at 178.8129 49.2322) (size 0.6) (drill 0.3) (layers "F.Cu" "B.Cu") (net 36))
 (segment (start 178.8129 93.2671) (end 178.8129 49.2322) (width 0.2) (layer "B.Cu") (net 36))
 (segment (start 181.5214 46.5237) (end 178.8129 49.2322) (width 0.2) (layer "B.Cu") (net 36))
 (segment (start 178.8129 49.2322) (end 181.5214 46.5237) (width 0.2) (layer "B.Cu") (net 36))
 (segment (start 177.5 94.58) (end 178.8129 93.2671) (width 0.2) (layer "B.Cu") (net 36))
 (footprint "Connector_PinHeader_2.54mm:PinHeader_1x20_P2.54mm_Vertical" (layer "F.Cu") (at 195.0 120.0)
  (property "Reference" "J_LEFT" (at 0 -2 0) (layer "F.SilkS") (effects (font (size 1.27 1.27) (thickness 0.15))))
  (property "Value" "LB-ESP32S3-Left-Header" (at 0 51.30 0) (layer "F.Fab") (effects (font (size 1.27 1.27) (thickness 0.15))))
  (pad "1" thru_hole rect (at 0 0.00) (size 1.7 1.7) (drill 1) (layers "*.Cu" "*.Mask") (remove_unused_layers no) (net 48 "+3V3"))
  (pad "2" thru_hole circle (at 0 2.54) (size 1.7 1.7) (drill 1) (layers "*.Cu" "*.Mask") (remove_unused_layers no) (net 48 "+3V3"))
  (pad "3" thru_hole circle (at 0 5.08) (size 1.7 1.7) (drill 1) (layers "*.Cu" "*.Mask") (remove_unused_layers no) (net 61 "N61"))
  (pad "4" thru_hole circle (at 0 7.62) (size 1.7 1.7) (drill 1) (layers "*.Cu" "*.Mask") (remove_unused_layers no) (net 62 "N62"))
  (pad "5" thru_hole circle (at 0 10.16) (size 1.7 1.7) (drill 1) (layers "*.Cu" "*.Mask") (remove_unused_layers no) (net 37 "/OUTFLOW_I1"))
  (pad "6" thru_hole circle (at 0 12.70) (size 1.7 1.7) (drill 1) (layers "*.Cu" "*.Mask") (remove_unused_layers no) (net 20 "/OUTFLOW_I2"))
  (pad "7" thru_hole circle (at 0 15.24) (size 1.7 1.7) (drill 1) (layers "*.Cu" "*.Mask") (remove_unused_layers no) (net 21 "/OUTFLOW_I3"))
  (pad "8" thru_hole circle (at 0 17.78) (size 1.7 1.7) (drill 1) (layers "*.Cu" "*.Mask") (remove_unused_layers no) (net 22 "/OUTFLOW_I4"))
  (pad "9" thru_hole circle (at 0 20.32) (size 1.7 1.7) (drill 1) (layers "*.Cu" "*.Mask") (remove_unused_layers no) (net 32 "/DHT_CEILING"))
  (pad "10" thru_hole circle (at 0 22.86) (size 1.7 1.7) (drill 1) (layers "*.Cu" "*.Mask") (remove_unused_layers no) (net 33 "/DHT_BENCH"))
  (pad "11" thru_hole circle (at 0 25.40) (size 1.7 1.7) (drill 1) (layers "*.Cu" "*.Mask") (remove_unused_layers no) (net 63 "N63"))
  (pad "12" thru_hole circle (at 0 27.94) (size 1.7 1.7) (drill 1) (layers "*.Cu" "*.Mask") (remove_unused_layers no) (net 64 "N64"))
  (pad "13" thru_hole circle (at 0 30.48) (size 1.7 1.7) (drill 1) (layers "*.Cu" "*.Mask") (remove_unused_layers no) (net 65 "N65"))
  (pad "14" thru_hole circle (at 0 33.02) (size 1.7 1.7) (drill 1) (layers "*.Cu" "*.Mask") (remove_unused_layers no) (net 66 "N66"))
  (pad "15" thru_hole circle (at 0 35.56) (size 1.7 1.7) (drill 1) (layers "*.Cu" "*.Mask") (remove_unused_layers no) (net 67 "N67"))
  (pad "16" thru_hole circle (at 0 38.10) (size 1.7 1.7) (drill 1) (layers "*.Cu" "*.Mask") (remove_unused_layers no) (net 12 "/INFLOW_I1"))
  (pad "17" thru_hole circle (at 0 40.64) (size 1.7 1.7) (drill 1) (layers "*.Cu" "*.Mask") (remove_unused_layers no) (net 11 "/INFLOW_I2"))
  (pad "18" thru_hole circle (at 0 43.18) (size 1.7 1.7) (drill 1) (layers "*.Cu" "*.Mask") (remove_unused_layers no) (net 10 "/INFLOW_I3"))
  (pad "19" thru_hole circle (at 0 45.72) (size 1.7 1.7) (drill 1) (layers "*.Cu" "*.Mask") (remove_unused_layers no) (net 9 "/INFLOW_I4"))
  (pad "20" thru_hole circle (at 0 48.26) (size 1.7 1.7) (drill 1) (layers "*.Cu" "*.Mask") (remove_unused_layers no) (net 50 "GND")))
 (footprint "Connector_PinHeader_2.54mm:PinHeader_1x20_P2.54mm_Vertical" (layer "F.Cu") (at 205.0 120.0)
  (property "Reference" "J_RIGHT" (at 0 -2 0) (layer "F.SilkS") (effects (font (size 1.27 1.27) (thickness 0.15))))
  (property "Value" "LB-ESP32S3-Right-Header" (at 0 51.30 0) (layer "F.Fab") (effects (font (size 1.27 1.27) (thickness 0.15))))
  (pad "1" thru_hole rect (at 0 0.00) (size 1.7 1.7) (drill 1) (layers "*.Cu" "*.Mask") (remove_unused_layers no) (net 50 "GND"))
  (pad "2" thru_hole circle (at 0 2.54) (size 1.7 1.7) (drill 1) (layers "*.Cu" "*.Mask") (remove_unused_layers no) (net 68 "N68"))
  (pad "3" thru_hole circle (at 0 5.08) (size 1.7 1.7) (drill 1) (layers "*.Cu" "*.Mask") (remove_unused_layers no) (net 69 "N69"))
  (pad "4" thru_hole circle (at 0 7.62) (size 1.7 1.7) (drill 1) (layers "*.Cu" "*.Mask") (remove_unused_layers no) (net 31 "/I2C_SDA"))
  (pad "5" thru_hole circle (at 0 10.16) (size 1.7 1.7) (drill 1) (layers "*.Cu" "*.Mask") (remove_unused_layers no) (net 24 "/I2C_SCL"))
  (pad "6" thru_hole circle (at 0 12.70) (size 1.7 1.7) (drill 1) (layers "*.Cu" "*.Mask") (remove_unused_layers no) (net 34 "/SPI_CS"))
  (pad "7" thru_hole circle (at 0 15.24) (size 1.7 1.7) (drill 1) (layers "*.Cu" "*.Mask") (remove_unused_layers no) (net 35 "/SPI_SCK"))
  (pad "8" thru_hole circle (at 0 17.78) (size 1.7 1.7) (drill 1) (layers "*.Cu" "*.Mask") (remove_unused_layers no) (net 36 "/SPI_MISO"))
  (pad "9" thru_hole circle (at 0 20.32) (size 1.7 1.7) (drill 1) (layers "*.Cu" "*.Mask") (remove_unused_layers no) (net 40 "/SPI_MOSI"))
  (pad "10" thru_hole circle (at 0 22.86) (size 1.7 1.7) (drill 1) (layers "*.Cu" "*.Mask") (remove_unused_layers no) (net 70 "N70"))
  (pad "11" thru_hole circle (at 0 25.40) (size 1.7 1.7) (drill 1) (layers "*.Cu" "*.Mask") (remove_unused_layers no) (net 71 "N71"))
  (pad "12" thru_hole circle (at 0 27.94) (size 1.7 1.7) (drill 1) (layers "*.Cu" "*.Mask") (remove_unused_layers no) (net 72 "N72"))
  (pad "13" thru_hole circle (at 0 30.48) (size 1.7 1.7) (drill 1) (layers "*.Cu" "*.Mask") (remove_unused_layers no) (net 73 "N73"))
  (pad "14" thru_hole circle (at 0 33.02) (size 1.7 1.7) (drill 1) (layers "*.Cu" "*.Mask") (remove_unused_layers no) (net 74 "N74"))
  (pad "15" thru_hole circle (at 0 35.56) (size 1.7 1.7) (drill 1) (layers "*.Cu" "*.Mask") (remove_unused_layers no) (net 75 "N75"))
  (pad "16" thru_hole circle (at 0 38.10) (size 1.7 1.7) (drill 1) (layers "*.Cu" "*.Mask") (remove_unused_layers no) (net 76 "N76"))
  (pad "17" thru_hole circle (at 0 40.64) (size 1.7 1.7) (drill 1) (layers "*.Cu" "*.Mask") (remove_unused_layers no) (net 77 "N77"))
  (pad "18" thru_hole circle (at 0 43.18) (size 1.7 1.7) (drill 1) (layers "*.Cu" "*.Mask") (remove_unused_layers no) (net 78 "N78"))
  (pad "19" thru_hole circle (at 0 45.72) (size 1.7 1.7) (drill 1) (layers "*.Cu" "*.Mask") (remove_unused_layers no) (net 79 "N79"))
  (pad "20" thru_hole circle (at 0 48.26) (size 1.7 1.7) (drill 1) (layers "*.Cu" "*.Mask") (remove_unused_layers no) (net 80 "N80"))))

